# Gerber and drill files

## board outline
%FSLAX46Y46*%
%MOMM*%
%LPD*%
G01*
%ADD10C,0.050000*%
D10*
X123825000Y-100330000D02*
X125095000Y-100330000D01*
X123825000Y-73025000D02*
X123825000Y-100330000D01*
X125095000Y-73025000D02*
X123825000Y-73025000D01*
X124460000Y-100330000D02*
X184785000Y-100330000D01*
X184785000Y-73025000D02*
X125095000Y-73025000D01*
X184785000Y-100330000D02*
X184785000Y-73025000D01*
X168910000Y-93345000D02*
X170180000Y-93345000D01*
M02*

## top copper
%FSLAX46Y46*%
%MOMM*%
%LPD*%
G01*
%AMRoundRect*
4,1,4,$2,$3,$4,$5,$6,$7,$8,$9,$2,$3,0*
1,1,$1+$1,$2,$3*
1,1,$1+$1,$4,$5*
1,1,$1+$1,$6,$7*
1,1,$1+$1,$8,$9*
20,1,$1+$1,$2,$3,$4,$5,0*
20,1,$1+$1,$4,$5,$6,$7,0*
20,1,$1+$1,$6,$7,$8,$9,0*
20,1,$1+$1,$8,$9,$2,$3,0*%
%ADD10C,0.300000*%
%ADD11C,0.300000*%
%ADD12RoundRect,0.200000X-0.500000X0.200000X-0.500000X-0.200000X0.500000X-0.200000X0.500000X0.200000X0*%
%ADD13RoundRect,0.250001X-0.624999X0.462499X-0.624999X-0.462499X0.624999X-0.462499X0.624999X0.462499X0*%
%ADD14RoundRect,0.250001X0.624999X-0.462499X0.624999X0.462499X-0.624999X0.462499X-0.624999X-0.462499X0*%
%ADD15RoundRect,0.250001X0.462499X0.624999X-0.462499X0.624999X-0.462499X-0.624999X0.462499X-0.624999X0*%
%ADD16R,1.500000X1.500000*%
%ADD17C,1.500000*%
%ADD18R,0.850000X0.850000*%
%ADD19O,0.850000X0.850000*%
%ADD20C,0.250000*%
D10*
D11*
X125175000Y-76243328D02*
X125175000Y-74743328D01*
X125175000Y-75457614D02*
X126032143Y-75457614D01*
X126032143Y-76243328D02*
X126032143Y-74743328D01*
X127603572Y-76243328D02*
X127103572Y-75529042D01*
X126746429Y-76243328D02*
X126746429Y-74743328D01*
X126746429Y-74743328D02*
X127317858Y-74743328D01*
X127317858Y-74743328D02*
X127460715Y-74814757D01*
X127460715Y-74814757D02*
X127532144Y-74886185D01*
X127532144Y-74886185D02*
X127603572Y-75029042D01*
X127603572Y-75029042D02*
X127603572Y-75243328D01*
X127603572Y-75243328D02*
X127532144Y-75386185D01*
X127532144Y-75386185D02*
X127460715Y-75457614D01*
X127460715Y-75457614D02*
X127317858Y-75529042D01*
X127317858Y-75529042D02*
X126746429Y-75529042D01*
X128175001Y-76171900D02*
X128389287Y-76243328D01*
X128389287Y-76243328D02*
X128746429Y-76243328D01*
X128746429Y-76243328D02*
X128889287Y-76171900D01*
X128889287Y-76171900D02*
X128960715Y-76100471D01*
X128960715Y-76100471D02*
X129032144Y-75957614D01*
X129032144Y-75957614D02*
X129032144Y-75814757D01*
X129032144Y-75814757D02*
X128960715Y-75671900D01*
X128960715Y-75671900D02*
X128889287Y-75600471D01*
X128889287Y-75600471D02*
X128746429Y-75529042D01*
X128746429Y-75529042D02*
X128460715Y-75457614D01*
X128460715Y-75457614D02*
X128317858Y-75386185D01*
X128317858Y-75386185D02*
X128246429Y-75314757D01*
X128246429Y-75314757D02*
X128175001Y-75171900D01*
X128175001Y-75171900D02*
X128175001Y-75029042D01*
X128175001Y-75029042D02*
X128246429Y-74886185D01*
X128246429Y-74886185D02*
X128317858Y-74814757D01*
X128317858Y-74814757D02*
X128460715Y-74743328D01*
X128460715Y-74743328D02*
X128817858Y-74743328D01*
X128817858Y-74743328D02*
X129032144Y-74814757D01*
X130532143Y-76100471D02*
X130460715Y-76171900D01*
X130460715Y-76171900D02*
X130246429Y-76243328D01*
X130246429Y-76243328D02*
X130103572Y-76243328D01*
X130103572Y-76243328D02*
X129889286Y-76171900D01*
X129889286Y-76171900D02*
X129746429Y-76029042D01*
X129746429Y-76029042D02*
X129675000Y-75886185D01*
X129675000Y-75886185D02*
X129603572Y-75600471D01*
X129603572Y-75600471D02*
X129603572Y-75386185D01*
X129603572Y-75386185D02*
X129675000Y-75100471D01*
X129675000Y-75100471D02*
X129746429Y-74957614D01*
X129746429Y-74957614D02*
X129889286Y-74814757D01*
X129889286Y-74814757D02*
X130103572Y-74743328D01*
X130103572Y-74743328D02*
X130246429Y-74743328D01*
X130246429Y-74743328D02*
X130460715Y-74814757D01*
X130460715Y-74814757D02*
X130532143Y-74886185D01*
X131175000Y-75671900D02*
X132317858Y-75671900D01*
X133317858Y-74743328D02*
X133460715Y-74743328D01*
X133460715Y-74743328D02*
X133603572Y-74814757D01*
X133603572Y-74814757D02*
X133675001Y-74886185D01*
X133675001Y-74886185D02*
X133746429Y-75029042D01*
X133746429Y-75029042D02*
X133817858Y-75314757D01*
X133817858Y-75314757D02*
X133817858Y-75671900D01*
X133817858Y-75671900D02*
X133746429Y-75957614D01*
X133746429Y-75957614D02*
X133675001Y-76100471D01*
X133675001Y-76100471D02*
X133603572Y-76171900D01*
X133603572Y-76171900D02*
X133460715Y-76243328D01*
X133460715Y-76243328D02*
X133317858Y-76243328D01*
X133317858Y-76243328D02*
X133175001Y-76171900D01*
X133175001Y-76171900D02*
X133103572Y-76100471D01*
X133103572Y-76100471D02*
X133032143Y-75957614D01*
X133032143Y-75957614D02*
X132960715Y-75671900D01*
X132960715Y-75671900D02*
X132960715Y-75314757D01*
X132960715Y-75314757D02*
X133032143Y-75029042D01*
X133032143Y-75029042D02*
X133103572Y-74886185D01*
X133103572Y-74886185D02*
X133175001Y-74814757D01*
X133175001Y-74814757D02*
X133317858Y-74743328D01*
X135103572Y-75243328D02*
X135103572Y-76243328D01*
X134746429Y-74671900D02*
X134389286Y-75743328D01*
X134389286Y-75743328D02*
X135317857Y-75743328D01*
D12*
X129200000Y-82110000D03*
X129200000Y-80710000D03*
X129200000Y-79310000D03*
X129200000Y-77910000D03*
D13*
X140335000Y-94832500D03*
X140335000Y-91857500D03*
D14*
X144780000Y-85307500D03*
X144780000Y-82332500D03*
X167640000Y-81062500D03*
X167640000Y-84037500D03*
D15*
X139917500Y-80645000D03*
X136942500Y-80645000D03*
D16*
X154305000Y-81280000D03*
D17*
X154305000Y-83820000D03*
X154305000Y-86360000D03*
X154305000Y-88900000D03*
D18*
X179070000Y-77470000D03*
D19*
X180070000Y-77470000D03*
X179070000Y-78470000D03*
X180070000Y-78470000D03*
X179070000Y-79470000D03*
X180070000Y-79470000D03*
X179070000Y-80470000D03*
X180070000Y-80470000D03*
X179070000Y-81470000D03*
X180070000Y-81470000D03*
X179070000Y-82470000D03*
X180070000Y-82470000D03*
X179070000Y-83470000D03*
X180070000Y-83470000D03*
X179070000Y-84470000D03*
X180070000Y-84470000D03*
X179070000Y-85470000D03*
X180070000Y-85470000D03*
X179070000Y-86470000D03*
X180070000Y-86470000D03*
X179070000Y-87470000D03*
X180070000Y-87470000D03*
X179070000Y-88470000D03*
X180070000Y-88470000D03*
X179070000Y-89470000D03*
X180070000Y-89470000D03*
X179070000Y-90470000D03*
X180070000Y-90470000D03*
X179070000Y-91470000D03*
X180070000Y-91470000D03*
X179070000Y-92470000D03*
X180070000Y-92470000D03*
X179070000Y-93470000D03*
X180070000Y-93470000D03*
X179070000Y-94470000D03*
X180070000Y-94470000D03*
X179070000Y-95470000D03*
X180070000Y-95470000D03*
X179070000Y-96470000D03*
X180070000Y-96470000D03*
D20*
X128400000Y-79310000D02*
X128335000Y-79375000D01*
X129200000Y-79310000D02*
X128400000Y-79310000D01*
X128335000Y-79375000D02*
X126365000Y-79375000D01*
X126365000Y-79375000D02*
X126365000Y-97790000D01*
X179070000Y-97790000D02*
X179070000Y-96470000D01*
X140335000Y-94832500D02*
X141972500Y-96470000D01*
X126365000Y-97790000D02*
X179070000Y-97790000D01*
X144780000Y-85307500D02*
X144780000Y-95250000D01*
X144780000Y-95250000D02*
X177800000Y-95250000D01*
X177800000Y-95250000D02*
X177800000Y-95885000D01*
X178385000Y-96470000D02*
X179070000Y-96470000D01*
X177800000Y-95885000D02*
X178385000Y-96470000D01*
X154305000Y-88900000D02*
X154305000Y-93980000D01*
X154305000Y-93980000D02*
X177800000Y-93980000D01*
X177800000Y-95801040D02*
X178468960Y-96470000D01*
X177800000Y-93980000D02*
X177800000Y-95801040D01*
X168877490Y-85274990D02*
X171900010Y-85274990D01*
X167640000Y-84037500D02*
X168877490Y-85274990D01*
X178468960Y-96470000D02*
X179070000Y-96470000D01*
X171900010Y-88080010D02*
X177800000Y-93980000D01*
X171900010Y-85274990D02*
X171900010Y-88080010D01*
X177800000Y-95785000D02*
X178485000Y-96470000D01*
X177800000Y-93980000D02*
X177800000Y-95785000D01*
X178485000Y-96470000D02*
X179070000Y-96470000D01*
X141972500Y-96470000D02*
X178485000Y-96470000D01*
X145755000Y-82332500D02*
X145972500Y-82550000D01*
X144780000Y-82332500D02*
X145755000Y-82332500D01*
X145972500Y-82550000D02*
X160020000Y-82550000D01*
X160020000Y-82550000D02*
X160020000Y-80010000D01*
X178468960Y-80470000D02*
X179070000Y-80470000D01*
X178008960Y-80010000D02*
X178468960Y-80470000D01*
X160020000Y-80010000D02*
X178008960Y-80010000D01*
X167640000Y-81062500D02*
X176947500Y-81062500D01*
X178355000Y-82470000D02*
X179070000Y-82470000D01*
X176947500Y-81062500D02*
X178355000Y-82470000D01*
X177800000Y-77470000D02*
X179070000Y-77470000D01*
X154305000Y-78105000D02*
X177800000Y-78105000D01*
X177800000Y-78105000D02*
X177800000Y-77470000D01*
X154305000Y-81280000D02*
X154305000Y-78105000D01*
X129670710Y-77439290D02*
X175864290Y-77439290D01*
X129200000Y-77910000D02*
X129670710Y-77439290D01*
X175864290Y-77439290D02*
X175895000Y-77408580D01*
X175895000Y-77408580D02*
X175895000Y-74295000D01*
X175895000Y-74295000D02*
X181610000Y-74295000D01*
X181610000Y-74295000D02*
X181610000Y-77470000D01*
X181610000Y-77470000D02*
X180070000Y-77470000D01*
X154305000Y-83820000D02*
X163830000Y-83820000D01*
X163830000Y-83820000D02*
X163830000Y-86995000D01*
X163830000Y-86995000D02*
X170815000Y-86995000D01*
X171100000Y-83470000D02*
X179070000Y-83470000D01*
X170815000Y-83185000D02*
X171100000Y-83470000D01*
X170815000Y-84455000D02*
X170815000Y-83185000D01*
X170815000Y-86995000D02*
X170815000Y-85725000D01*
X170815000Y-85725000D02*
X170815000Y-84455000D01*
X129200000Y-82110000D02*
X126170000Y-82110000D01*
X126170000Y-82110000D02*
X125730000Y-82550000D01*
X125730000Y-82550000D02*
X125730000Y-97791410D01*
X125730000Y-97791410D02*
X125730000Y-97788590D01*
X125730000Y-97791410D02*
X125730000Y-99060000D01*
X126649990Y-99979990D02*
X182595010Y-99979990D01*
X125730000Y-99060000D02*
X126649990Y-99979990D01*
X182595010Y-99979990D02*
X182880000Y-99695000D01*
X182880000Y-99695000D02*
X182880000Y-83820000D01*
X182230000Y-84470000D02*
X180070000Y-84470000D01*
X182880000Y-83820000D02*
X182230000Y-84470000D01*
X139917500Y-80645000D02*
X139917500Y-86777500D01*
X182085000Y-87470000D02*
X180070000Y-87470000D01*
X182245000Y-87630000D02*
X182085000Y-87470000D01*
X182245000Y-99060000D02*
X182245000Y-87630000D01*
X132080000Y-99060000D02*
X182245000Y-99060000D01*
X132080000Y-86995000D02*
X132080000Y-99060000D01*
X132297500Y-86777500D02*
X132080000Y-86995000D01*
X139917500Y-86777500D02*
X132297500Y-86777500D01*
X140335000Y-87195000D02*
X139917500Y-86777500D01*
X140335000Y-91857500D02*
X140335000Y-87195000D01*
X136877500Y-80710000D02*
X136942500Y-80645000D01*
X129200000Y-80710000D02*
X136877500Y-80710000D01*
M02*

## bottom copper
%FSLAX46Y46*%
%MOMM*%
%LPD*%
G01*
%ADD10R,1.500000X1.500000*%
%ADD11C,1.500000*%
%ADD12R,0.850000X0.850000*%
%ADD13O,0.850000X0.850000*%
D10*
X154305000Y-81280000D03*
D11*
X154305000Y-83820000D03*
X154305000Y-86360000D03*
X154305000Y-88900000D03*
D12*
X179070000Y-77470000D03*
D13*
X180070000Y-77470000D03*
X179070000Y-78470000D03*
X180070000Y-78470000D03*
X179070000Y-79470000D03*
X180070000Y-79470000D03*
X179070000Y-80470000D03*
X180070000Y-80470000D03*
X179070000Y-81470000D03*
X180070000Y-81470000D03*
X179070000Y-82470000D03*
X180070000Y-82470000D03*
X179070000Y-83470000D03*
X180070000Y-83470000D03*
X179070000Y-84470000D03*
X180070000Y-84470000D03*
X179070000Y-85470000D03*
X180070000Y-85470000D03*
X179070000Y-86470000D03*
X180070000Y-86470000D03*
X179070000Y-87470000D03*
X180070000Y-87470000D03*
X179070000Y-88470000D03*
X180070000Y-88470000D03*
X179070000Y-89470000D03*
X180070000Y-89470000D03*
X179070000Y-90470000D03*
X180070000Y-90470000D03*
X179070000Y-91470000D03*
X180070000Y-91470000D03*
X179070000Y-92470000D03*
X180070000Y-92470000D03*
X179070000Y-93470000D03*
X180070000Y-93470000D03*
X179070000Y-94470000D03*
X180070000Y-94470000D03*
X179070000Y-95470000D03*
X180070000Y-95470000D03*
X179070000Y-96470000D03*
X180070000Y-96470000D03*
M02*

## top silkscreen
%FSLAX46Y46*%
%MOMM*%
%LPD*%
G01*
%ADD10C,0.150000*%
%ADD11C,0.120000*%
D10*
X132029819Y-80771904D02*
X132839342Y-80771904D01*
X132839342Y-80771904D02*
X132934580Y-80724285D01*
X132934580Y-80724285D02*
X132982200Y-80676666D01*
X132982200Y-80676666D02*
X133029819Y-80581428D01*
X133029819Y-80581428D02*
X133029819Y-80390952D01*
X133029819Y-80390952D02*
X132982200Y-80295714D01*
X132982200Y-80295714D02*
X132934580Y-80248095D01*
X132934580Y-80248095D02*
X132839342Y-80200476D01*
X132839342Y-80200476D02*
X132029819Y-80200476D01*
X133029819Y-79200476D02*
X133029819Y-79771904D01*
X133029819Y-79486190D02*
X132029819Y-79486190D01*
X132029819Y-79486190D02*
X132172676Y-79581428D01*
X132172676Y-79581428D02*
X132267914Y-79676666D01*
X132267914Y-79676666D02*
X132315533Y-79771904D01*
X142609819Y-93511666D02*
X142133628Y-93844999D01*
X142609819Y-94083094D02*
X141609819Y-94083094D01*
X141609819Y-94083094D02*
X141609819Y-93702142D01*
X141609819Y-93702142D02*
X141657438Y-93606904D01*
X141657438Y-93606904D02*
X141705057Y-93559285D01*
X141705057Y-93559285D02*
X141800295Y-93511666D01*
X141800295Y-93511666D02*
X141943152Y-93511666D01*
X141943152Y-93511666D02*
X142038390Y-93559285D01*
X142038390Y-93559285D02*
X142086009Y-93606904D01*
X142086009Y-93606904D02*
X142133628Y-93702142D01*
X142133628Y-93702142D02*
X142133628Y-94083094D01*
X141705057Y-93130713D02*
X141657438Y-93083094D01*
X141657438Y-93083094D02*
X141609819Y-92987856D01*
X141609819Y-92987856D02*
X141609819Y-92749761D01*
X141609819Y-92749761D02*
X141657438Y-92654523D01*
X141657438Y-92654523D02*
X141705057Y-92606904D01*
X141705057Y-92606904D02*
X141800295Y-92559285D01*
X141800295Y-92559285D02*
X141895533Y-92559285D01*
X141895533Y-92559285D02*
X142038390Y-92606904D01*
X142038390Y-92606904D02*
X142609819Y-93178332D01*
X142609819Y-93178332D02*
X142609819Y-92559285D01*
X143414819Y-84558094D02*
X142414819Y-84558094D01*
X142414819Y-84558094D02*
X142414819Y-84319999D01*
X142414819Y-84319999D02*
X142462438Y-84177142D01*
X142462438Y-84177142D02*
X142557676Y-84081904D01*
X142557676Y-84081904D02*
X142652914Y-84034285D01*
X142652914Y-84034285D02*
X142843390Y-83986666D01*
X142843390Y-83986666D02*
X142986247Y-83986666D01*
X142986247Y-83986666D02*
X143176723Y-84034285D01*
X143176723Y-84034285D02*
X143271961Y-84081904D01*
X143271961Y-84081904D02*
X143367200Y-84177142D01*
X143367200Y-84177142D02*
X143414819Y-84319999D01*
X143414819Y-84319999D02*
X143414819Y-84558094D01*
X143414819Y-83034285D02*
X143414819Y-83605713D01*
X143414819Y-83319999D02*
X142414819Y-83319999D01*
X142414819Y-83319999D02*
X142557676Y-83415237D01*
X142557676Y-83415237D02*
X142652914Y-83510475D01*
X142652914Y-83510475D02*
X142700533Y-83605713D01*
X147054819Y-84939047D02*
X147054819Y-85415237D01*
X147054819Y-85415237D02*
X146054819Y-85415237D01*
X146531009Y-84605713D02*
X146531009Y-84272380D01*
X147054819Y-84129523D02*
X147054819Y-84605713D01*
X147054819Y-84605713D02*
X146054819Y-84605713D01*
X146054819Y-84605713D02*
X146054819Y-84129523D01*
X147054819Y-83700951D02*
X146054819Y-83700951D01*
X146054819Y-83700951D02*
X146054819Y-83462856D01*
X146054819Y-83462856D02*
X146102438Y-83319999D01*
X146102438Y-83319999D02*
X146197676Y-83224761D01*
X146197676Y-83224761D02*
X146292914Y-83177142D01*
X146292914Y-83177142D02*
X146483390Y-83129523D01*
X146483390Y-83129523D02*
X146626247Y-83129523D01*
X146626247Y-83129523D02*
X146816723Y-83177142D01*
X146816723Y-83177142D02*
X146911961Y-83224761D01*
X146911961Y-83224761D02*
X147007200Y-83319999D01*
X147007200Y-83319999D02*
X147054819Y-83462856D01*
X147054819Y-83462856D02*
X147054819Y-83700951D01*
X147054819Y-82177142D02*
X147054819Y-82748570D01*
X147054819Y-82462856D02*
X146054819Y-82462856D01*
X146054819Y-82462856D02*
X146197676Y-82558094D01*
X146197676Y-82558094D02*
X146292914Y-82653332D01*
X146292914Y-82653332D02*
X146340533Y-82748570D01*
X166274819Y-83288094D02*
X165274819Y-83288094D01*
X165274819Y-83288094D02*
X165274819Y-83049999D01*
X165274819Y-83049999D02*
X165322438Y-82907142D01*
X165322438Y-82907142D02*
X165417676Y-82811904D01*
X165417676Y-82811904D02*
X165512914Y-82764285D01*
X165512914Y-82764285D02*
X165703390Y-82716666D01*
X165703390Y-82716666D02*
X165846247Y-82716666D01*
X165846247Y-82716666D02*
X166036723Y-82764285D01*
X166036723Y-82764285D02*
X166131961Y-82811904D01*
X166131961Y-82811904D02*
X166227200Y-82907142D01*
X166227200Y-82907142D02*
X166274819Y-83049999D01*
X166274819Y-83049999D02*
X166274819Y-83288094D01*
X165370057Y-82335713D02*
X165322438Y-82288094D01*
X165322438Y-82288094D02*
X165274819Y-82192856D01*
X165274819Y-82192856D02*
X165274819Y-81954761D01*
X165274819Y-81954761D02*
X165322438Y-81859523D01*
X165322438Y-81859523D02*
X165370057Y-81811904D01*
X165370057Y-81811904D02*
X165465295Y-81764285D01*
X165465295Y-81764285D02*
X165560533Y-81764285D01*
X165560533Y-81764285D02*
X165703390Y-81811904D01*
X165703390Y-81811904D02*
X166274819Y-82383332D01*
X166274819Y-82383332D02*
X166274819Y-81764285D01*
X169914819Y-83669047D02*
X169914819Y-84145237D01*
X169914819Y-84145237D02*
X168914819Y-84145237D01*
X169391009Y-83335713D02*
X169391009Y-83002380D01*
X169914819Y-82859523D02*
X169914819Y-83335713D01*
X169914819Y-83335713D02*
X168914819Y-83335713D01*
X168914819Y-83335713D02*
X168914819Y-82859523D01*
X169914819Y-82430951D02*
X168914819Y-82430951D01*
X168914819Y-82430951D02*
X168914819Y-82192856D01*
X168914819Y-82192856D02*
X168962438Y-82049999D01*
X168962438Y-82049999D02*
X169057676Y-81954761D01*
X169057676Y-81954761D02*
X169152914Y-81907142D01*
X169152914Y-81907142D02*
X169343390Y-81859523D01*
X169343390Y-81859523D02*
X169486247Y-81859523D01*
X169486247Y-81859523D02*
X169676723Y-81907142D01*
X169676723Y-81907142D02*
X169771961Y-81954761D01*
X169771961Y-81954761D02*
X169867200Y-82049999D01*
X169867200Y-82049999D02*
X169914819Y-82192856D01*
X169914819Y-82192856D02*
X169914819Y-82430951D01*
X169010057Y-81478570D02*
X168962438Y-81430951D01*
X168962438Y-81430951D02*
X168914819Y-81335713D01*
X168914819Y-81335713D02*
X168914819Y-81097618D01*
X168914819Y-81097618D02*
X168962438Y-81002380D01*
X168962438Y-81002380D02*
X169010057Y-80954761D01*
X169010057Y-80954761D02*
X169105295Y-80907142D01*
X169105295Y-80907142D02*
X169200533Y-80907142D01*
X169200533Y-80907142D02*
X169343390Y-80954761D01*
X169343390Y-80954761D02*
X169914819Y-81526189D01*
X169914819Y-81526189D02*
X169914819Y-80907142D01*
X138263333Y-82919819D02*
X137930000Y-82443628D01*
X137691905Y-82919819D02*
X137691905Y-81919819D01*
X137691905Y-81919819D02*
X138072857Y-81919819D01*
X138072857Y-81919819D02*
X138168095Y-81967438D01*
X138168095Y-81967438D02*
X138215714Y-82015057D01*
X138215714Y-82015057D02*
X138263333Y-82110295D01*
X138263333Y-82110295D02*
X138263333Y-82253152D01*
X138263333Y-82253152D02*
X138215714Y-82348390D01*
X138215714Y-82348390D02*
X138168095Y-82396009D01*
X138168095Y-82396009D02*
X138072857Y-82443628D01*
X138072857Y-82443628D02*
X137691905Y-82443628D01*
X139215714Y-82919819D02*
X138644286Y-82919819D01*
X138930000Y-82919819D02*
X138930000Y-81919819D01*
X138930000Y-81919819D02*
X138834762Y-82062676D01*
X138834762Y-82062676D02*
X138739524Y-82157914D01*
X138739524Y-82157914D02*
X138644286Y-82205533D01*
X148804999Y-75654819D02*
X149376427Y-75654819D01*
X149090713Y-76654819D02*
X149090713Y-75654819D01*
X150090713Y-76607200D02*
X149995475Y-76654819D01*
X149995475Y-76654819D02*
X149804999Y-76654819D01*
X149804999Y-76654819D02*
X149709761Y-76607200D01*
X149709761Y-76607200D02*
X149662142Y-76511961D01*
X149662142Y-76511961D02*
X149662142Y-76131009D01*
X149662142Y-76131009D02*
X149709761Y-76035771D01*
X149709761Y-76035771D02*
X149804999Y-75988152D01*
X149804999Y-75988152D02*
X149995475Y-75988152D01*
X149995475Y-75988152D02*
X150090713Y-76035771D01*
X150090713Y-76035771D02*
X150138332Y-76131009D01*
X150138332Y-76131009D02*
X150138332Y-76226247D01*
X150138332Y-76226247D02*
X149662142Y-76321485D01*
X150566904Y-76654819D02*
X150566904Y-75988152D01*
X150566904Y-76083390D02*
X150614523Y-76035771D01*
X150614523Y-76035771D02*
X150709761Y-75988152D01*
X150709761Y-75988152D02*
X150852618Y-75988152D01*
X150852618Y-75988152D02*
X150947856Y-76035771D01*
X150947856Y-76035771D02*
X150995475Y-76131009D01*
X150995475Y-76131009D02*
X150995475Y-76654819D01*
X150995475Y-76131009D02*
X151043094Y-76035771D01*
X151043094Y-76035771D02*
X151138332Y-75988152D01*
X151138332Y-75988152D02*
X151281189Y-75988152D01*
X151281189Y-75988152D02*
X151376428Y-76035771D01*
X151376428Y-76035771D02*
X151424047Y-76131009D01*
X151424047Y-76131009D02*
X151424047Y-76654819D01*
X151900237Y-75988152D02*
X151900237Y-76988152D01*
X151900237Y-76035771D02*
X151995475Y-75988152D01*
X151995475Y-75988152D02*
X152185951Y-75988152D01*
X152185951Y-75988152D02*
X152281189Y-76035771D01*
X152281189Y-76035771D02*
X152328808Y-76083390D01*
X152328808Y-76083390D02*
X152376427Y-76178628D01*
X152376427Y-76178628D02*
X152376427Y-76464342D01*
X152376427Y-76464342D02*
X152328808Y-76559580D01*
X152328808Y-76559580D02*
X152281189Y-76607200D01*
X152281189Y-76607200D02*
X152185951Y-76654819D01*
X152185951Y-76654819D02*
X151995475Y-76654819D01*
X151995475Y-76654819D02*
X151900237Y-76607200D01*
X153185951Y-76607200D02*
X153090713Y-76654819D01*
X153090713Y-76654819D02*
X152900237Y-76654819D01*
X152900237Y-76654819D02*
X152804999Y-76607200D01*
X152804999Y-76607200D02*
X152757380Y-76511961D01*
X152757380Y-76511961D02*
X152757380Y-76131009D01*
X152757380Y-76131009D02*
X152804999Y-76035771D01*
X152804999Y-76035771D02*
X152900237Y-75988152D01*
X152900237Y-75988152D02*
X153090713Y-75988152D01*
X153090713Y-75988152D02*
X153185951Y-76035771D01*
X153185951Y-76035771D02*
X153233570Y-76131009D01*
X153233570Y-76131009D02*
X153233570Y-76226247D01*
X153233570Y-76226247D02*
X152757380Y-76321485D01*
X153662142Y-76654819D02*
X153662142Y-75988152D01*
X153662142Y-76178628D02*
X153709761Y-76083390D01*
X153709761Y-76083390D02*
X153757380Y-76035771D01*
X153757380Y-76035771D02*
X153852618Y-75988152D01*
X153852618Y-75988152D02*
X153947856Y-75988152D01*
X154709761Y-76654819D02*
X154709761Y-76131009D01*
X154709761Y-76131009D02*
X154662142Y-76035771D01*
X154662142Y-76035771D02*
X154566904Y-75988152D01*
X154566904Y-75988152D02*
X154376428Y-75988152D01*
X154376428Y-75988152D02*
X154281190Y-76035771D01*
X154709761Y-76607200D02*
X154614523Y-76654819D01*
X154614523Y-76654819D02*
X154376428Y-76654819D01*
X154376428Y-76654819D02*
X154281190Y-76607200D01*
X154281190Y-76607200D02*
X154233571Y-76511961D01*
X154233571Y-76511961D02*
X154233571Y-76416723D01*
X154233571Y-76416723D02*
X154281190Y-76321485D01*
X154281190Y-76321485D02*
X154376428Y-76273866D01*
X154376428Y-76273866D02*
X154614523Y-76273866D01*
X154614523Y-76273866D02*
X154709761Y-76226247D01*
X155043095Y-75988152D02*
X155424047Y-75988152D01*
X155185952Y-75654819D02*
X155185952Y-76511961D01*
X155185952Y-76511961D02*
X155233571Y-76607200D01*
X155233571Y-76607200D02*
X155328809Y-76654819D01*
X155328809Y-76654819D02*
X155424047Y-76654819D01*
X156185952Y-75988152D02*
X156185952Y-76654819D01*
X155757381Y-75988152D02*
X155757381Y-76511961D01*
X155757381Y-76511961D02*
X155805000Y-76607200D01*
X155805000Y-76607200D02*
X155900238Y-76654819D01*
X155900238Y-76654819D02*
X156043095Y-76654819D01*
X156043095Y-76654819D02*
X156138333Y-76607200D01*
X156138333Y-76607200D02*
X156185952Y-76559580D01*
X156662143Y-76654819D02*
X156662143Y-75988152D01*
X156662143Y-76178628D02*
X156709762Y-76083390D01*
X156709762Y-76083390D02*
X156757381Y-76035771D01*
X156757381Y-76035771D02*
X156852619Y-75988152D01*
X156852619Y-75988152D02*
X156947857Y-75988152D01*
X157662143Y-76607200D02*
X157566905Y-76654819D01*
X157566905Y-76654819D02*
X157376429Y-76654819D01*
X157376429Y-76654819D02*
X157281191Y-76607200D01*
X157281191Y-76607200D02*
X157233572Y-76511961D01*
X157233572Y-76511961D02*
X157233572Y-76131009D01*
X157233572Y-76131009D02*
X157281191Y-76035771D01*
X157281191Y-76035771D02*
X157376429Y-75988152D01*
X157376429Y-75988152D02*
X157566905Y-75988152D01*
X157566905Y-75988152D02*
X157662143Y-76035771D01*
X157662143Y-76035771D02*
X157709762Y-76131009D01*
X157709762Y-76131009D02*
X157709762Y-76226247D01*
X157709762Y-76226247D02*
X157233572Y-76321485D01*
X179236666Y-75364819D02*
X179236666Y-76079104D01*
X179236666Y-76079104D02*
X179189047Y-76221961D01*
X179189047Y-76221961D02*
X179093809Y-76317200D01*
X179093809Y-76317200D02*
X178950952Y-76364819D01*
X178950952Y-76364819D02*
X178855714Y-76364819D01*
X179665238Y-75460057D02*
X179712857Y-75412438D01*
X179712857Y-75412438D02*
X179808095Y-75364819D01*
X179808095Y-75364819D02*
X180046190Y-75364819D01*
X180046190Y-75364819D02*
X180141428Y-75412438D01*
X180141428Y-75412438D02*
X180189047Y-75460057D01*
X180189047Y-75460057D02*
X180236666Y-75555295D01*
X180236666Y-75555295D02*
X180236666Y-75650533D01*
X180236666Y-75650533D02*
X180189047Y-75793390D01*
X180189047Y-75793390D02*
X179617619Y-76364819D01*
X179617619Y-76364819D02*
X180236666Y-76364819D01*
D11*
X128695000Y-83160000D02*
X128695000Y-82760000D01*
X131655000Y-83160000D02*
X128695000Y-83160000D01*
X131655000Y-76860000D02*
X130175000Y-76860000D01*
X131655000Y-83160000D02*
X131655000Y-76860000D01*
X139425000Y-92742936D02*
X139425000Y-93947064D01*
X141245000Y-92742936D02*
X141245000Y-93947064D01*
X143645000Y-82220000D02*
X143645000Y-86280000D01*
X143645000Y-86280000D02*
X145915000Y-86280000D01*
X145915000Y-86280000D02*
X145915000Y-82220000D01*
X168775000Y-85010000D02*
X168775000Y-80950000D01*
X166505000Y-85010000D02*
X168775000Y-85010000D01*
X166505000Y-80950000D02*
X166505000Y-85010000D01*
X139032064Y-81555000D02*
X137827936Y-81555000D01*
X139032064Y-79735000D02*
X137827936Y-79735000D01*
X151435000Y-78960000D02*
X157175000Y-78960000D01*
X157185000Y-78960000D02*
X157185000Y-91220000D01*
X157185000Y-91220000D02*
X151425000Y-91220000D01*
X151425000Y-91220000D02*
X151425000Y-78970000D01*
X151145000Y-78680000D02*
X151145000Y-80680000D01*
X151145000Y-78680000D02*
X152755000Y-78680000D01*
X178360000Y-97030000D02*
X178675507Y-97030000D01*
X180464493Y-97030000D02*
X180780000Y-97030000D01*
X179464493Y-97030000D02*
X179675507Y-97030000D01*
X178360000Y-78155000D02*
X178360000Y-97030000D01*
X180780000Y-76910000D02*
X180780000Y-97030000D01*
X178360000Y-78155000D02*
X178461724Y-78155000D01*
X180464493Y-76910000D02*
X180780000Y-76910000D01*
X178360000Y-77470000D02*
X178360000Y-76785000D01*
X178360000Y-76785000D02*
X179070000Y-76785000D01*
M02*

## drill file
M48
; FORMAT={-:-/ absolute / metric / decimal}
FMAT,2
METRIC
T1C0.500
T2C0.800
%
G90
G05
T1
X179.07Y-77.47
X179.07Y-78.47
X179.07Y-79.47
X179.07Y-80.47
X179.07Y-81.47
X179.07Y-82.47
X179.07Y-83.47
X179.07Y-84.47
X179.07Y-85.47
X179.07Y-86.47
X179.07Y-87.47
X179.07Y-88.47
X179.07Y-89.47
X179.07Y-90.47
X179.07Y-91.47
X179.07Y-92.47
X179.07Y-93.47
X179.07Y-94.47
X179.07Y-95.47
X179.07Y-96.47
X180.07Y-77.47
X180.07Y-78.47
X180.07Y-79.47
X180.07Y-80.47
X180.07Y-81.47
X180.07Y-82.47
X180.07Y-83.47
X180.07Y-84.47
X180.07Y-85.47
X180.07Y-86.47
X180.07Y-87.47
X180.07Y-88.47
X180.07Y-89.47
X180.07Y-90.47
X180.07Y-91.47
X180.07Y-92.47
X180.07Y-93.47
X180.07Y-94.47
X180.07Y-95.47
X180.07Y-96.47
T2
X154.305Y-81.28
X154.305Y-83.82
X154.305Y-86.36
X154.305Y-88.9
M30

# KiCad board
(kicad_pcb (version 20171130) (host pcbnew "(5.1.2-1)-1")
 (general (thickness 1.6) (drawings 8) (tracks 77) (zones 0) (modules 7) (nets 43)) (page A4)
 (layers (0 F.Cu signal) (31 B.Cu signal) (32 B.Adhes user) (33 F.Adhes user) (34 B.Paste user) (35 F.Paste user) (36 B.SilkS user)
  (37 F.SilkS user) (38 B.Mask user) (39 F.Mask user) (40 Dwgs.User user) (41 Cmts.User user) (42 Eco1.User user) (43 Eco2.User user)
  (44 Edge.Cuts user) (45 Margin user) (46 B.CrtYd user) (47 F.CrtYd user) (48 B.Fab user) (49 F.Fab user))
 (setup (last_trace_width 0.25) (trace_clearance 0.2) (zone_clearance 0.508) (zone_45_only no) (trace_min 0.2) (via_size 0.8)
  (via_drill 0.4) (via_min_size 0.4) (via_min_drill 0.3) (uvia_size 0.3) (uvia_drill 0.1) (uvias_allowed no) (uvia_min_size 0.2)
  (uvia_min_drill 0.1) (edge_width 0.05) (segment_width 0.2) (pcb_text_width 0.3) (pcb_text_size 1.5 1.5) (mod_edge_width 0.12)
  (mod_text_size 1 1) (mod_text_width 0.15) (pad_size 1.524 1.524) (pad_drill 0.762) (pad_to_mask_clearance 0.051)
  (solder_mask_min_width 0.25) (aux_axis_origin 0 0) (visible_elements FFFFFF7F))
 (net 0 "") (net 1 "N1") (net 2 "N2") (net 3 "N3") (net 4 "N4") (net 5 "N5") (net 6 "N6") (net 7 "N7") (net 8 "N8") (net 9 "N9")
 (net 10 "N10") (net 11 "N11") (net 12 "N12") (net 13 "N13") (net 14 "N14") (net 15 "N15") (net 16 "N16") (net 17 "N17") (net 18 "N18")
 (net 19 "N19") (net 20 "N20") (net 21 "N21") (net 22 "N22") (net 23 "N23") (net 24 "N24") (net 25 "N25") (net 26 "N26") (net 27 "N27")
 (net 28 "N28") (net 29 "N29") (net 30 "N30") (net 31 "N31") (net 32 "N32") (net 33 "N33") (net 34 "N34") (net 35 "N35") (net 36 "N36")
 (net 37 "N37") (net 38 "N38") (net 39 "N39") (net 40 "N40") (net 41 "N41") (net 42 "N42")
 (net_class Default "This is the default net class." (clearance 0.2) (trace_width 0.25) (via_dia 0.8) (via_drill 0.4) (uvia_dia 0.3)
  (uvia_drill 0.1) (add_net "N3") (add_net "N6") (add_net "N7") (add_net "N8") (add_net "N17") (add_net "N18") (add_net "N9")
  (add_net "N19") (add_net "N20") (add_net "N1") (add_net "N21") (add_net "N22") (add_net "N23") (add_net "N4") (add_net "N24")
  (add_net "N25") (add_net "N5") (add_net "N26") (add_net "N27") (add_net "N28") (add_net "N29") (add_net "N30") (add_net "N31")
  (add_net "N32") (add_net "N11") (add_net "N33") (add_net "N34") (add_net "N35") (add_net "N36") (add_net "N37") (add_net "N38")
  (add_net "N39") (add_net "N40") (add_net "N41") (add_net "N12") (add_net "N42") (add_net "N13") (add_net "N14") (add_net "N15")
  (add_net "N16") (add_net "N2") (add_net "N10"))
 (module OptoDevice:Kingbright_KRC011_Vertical (layer F.Cu) (at 130.175 80.01 270)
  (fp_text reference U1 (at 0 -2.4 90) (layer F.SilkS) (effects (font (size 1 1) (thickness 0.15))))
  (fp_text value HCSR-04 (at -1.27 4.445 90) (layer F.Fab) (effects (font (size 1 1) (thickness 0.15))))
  (fp_line (start 3.15 1.48) (end 2.75 1.48) (layer F.SilkS) (width 0.12))
  (fp_line (start 3.15 -1.48) (end 3.15 1.48) (layer F.SilkS) (width 0.12))
  (fp_line (start -3.15 -1.48) (end -3.15 0) (layer F.SilkS) (width 0.12))
  (fp_line (start 3.15 -1.48) (end -3.15 -1.48) (layer F.SilkS) (width 0.12))
  (pad 4 smd roundrect (at 2.1 0.975 270) (size 0.8 1.4) (layers F.Cu F.Paste F.Mask) (roundrect_rratio 0.25) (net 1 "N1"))
  (pad 3 smd roundrect (at 0.7 0.975 270) (size 0.8 1.4) (layers F.Cu F.Paste F.Mask) (roundrect_rratio 0.25) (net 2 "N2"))
  (pad 2 smd roundrect (at -0.7 0.975 270) (size 0.8 1.4) (layers F.Cu F.Paste F.Mask) (roundrect_rratio 0.25) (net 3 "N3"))
  (pad 1 smd roundrect (at -2.1 0.975 270) (size 0.8 1.4) (layers F.Cu F.Paste F.Mask) (roundrect_rratio 0.25) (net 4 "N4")))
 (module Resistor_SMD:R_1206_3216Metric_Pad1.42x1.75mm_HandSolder (layer F.Cu) (at 140.335 93.345 270)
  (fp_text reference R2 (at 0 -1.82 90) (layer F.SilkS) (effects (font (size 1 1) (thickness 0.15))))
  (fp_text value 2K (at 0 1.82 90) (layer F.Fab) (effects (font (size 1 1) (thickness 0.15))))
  (fp_line (start -0.602064 0.91) (end 0.602064 0.91) (layer F.SilkS) (width 0.12))
  (fp_line (start -0.602064 -0.91) (end 0.602064 -0.91) (layer F.SilkS) (width 0.12))
  (pad 2 smd roundrect (at 1.4875 0 270) (size 1.425 1.75) (layers F.Cu F.Paste F.Mask) (roundrect_rratio 0.175439) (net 3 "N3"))
  (pad 1 smd roundrect (at -1.4875 0 270) (size 1.425 1.75) (layers F.Cu F.Paste F.Mask) (roundrect_rratio 0.175439) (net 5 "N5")))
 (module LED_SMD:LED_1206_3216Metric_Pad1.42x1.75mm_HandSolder (layer F.Cu) (at 144.78 83.82 90)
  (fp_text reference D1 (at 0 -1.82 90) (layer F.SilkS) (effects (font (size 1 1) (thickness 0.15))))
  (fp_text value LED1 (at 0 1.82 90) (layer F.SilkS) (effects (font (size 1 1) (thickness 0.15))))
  (fp_line (start 1.6 -1.135) (end -2.46 -1.135) (layer F.SilkS) (width 0.12))
  (fp_line (start -2.46 -1.135) (end -2.46 1.135) (layer F.SilkS) (width 0.12))
  (fp_line (start -2.46 1.135) (end 1.6 1.135) (layer F.SilkS) (width 0.12))
  (pad 1 smd roundrect (at -1.4875 0 90) (size 1.425 1.75) (layers F.Cu F.Paste F.Mask) (roundrect_rratio 0.175439) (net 3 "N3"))
  (pad 2 smd roundrect (at 1.4875 0 90) (size 1.425 1.75) (layers F.Cu F.Paste F.Mask) (roundrect_rratio 0.175439) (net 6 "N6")))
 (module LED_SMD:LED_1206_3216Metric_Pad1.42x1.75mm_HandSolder (layer F.Cu) (at 167.64 82.55 90)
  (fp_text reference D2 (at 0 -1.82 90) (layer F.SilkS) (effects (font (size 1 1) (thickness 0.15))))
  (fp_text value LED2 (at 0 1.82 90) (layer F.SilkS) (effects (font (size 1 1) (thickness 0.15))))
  (fp_line (start -2.46 1.135) (end 1.6 1.135) (layer F.SilkS) (width 0.12))
  (fp_line (start -2.46 -1.135) (end -2.46 1.135) (layer F.SilkS) (width 0.12))
  (fp_line (start 1.6 -1.135) (end -2.46 -1.135) (layer F.SilkS) (width 0.12))
  (pad 2 smd roundrect (at 1.4875 0 90) (size 1.425 1.75) (layers F.Cu F.Paste F.Mask) (roundrect_rratio 0.175439) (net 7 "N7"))
  (pad 1 smd roundrect (at -1.4875 0 90) (size 1.425 1.75) (layers F.Cu F.Paste F.Mask) (roundrect_rratio 0.175439) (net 3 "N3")))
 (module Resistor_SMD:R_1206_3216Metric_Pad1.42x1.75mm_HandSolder (layer F.Cu) (at 138.43 80.645 180)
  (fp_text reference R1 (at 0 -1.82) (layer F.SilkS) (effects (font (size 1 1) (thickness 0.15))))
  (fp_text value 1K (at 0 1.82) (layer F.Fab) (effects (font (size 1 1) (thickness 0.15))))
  (fp_line (start -0.602064 -0.91) (end 0.602064 -0.91) (layer F.SilkS) (width 0.12))
  (fp_line (start -0.602064 0.91) (end 0.602064 0.91) (layer F.SilkS) (width 0.12))
  (pad 1 smd roundrect (at -1.4875 0 180) (size 1.425 1.75) (layers F.Cu F.Paste F.Mask) (roundrect_rratio 0.175439) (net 5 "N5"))
  (pad 2 smd roundrect (at 1.4875 0 180) (size 1.425 1.75) (layers F.Cu F.Paste F.Mask) (roundrect_rratio 0.175439) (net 2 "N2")))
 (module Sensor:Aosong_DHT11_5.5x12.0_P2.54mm (layer F.Cu) (at 154.305 81.28)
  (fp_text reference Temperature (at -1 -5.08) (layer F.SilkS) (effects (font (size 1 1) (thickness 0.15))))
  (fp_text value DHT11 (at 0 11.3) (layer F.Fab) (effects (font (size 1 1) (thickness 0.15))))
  (fp_line (start -2.87 -2.32) (end 2.87 -2.32) (layer F.SilkS) (width 0.12))
  (fp_line (start 2.88 -2.32) (end 2.88 9.94) (layer F.SilkS) (width 0.12))
  (fp_line (start 2.88 9.94) (end -2.88 9.94) (layer F.SilkS) (width 0.12))
  (fp_line (start -2.88 9.94) (end -2.88 -2.31) (layer F.SilkS) (width 0.12))
  (fp_line (start -3.16 -2.6) (end -3.16 -0.6) (layer F.SilkS) (width 0.12))
  (fp_line (start -3.16 -2.6) (end -1.55 -2.6) (layer F.SilkS) (width 0.12))
  (pad 1 thru_hole rect (at 0 0) (size 1.5 1.5) (drill 0.8) (layers *.Cu *.Mask) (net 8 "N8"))
  (pad 2 thru_hole circle (at 0 2.54) (size 1.5 1.5) (drill 0.8) (layers *.Cu *.Mask) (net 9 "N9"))
  (pad 3 thru_hole circle (at 0 5.08) (size 1.5 1.5) (drill 0.8) (layers *.Cu *.Mask) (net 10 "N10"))
  (pad 4 thru_hole circle (at 0 7.62) (size 1.5 1.5) (drill 0.8) (layers *.Cu *.Mask) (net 3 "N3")))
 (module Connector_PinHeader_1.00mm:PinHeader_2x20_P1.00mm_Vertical (layer F.Cu) (at 179.07 77.47)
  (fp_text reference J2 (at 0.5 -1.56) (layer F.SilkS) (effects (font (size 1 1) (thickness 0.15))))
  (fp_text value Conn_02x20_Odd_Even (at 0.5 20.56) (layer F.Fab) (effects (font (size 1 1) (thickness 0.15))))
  (fp_line (start -0.71 19.56) (end -0.394493 19.56) (layer F.SilkS) (width 0.12))
  (fp_line (start 1.394493 19.56) (end 1.71 19.56) (layer F.SilkS) (width 0.12))
  (fp_line (start 0.394493 19.56) (end 0.605507 19.56) (layer F.SilkS) (width 0.12))
  (fp_line (start -0.71 0.685) (end -0.71 19.56) (layer F.SilkS) (width 0.12))
  (fp_line (start 1.71 -0.56) (end 1.71 19.56) (layer F.SilkS) (width 0.12))
  (fp_line (start -0.71 0.685) (end -0.608276 0.685) (layer F.SilkS) (width 0.12))
  (fp_line (start 1.394493 -0.56) (end 1.71 -0.56) (layer F.SilkS) (width 0.12))
  (fp_line (start -0.71 0) (end -0.71 -0.685) (layer F.SilkS) (width 0.12))
  (fp_line (start -0.71 -0.685) (end 0 -0.685) (layer F.SilkS) (width 0.12))
  (pad 1 thru_hole rect (at 0 0) (size 0.85 0.85) (drill 0.5) (layers *.Cu *.Mask) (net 8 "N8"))
  (pad 2 thru_hole oval (at 1 0) (size 0.85 0.85) (drill 0.5) (layers *.Cu *.Mask) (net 4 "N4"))
  (pad 3 thru_hole oval (at 0 1) (size 0.85 0.85) (drill 0.5) (layers *.Cu *.Mask) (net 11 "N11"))
  (pad 4 thru_hole oval (at 1 1) (size 0.85 0.85) (drill 0.5) (layers *.Cu *.Mask) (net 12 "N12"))
  (pad 5 thru_hole oval (at 0 2) (size 0.85 0.85) (drill 0.5) (layers *.Cu *.Mask) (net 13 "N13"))
  (pad 6 thru_hole oval (at 1 2) (size 0.85 0.85) (drill 0.5) (layers *.Cu *.Mask) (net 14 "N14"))
  (pad 7 thru_hole oval (at 0 3) (size 0.85 0.85) (drill 0.5) (layers *.Cu *.Mask) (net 6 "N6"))
  (pad 8 thru_hole oval (at 1 3) (size 0.85 0.85) (drill 0.5) (layers *.Cu *.Mask) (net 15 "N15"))
  (pad 9 thru_hole oval (at 0 4) (size 0.85 0.85) (drill 0.5) (layers *.Cu *.Mask) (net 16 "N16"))
  (pad 10 thru_hole oval (at 1 4) (size 0.85 0.85) (drill 0.5) (layers *.Cu *.Mask) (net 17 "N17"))
  (pad 11 thru_hole oval (at 0 5) (size 0.85 0.85) (drill 0.5) (layers *.Cu *.Mask) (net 7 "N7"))
  (pad 12 thru_hole oval (at 1 5) (size 0.85 0.85) (drill 0.5) (layers *.Cu *.Mask) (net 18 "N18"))
  (pad 13 thru_hole oval (at 0 6) (size 0.85 0.85) (drill 0.5) (layers *.Cu *.Mask) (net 9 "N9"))
  (pad 14 thru_hole oval (at 1 6) (size 0.85 0.85) (drill 0.5) (layers *.Cu *.Mask) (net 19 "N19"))
  (pad 15 thru_hole oval (at 0 7) (size 0.85 0.85) (drill 0.5) (layers *.Cu *.Mask) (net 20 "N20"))
  (pad 16 thru_hole oval (at 1 7) (size 0.85 0.85) (drill 0.5) (layers *.Cu *.Mask) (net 1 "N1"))
  (pad 17 thru_hole oval (at 0 8) (size 0.85 0.85) (drill 0.5) (layers *.Cu *.Mask) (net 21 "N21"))
  (pad 18 thru_hole oval (at 1 8) (size 0.85 0.85) (drill 0.5) (layers *.Cu *.Mask) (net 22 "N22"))
  (pad 19 thru_hole oval (at 0 9) (size 0.85 0.85) (drill 0.5) (layers *.Cu *.Mask) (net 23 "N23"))
  (pad 20 thru_hole oval (at 1 9) (size 0.85 0.85) (drill 0.5) (layers *.Cu *.Mask) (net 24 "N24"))
  (pad 21 thru_hole oval (at 0 10) (size 0.85 0.85) (drill 0.5) (layers *.Cu *.Mask) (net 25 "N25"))
  (pad 22 thru_hole oval (at 1 10) (size 0.85 0.85) (drill 0.5) (layers *.Cu *.Mask) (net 5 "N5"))
  (pad 23 thru_hole oval (at 0 11) (size 0.85 0.85) (drill 0.5) (layers *.Cu *.Mask) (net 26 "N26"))
  (pad 24 thru_hole oval (at 1 11) (size 0.85 0.85) (drill 0.5) (layers *.Cu *.Mask) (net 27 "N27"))
  (pad 25 thru_hole oval (at 0 12) (size 0.85 0.85) (drill 0.5) (layers *.Cu *.Mask) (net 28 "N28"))
  (pad 26 thru_hole oval (at 1 12) (size 0.85 0.85) (drill 0.5) (layers *.Cu *.Mask) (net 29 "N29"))
  (pad 27 thru_hole oval (at 0 13) (size 0.85 0.85) (drill 0.5) (layers *.Cu *.Mask) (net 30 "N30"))
  (pad 28 thru_hole oval (at 1 13) (size 0.85 0.85) (drill 0.5) (layers *.Cu *.Mask) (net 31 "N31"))
  (pad 29 thru_hole oval (at 0 14) (size 0.85 0.85) (drill 0.5) (layers *.Cu *.Mask) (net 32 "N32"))
  (pad 30 thru_hole oval (at 1 14) (size 0.85 0.85) (drill 0.5) (layers *.Cu *.Mask) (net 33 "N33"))
  (pad 31 thru_hole oval (at 0 15) (size 0.85 0.85) (drill 0.5) (layers *.Cu *.Mask) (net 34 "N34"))
  (pad 32 thru_hole oval (at 1 15) (size 0.85 0.85) (drill 0.5) (layers *.Cu *.Mask) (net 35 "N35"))
  (pad 33 thru_hole oval (at 0 16) (size 0.85 0.85) (drill 0.5) (layers *.Cu *.Mask) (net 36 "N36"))
  (pad 34 thru_hole oval (at 1 16) (size 0.85 0.85) (drill 0.5) (layers *.Cu *.Mask) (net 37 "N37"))
  (pad 35 thru_hole oval (at 0 17) (size 0.85 0.85) (drill 0.5) (layers *.Cu *.Mask) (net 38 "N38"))
  (pad 36 thru_hole oval (at 1 17) (size 0.85 0.85) (drill 0.5) (layers *.Cu *.Mask) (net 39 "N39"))
  (pad 37 thru_hole oval (at 0 18) (size 0.85 0.85) (drill 0.5) (layers *.Cu *.Mask) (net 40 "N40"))
  (pad 38 thru_hole oval (at 1 18) (size 0.85 0.85) (drill 0.5) (layers *.Cu *.Mask) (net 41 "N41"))
  (pad 39 thru_hole oval (at 0 19) (size 0.85 0.85) (drill 0.5) (layers *.Cu *.Mask) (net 3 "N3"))
  (pad 40 thru_hole oval (at 1 19) (size 0.85 0.85) (drill 0.5) (layers *.Cu *.Mask) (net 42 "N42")))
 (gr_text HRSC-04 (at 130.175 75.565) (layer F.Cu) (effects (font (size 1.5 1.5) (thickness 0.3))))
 (gr_line (start 123.825 100.33) (end 125.095 100.33) (layer Edge.Cuts) (width 0.05))
 (gr_line (start 123.825 73.025) (end 123.825 100.33) (layer Edge.Cuts) (width 0.05))
 (gr_line (start 125.095 73.025) (end 123.825 73.025) (layer Edge.Cuts) (width 0.05))
 (gr_line (start 124.46 100.33) (end 184.785 100.33) (layer Edge.Cuts) (width 0.05))
 (gr_line (start 184.785 73.025) (end 125.095 73.025) (layer Edge.Cuts) (width 0.05))
 (gr_line (start 184.785 100.33) (end 184.785 73.025) (layer Edge.Cuts) (width 0.05))
 (gr_line (start 168.91 93.345) (end 170.18 93.345) (layer Edge.Cuts) (width 0.05))
 (segment (start 128.4 79.31) (end 128.335 79.375) (width 0.25) (layer F.Cu) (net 3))
 (segment (start 129.2 79.31) (end 128.4 79.31) (width 0.25) (layer F.Cu) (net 3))
 (segment (start 128.335 79.375) (end 126.365 79.375) (width 0.25) (layer F.Cu) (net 3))
 (segment (start 126.365 79.375) (end 126.365 97.79) (width 0.25) (layer F.Cu) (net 3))
 (segment (start 179.07 97.79) (end 179.07 96.47) (width 0.25) (layer F.Cu) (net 3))
 (segment (start 140.335 94.8325) (end 141.9725 96.47) (width 0.25) (layer F.Cu) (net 3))
 (segment (start 126.365 97.79) (end 179.07 97.79) (width 0.25) (layer F.Cu) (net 3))
 (segment (start 144.78 85.3075) (end 144.78 95.25) (width 0.25) (layer F.Cu) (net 3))
 (segment (start 144.78 95.25) (end 177.8 95.25) (width 0.25) (layer F.Cu) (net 3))
 (segment (start 177.8 95.25) (end 177.8 95.885) (width 0.25) (layer F.Cu) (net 3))
 (segment (start 178.385 96.47) (end 179.07 96.47) (width 0.25) (layer F.Cu) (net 3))
 (segment (start 177.8 95.885) (end 178.385 96.47) (width 0.25) (layer F.Cu) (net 3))
 (segment (start 154.305 88.9) (end 154.305 93.98) (width 0.25) (layer F.Cu) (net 3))
 (segment (start 154.305 93.98) (end 177.8 93.98) (width 0.25) (layer F.Cu) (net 3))
 (segment (start 177.8 95.80104) (end 178.46896 96.47) (width 0.25) (layer F.Cu) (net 3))
 (segment (start 177.8 93.98) (end 177.8 95.80104) (width 0.25) (layer F.Cu) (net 3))
 (segment (start 168.87749 85.27499) (end 171.90001 85.27499) (width 0.25) (layer F.Cu) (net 3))
 (segment (start 167.64 84.0375) (end 168.87749 85.27499) (width 0.25) (layer F.Cu) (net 3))
 (segment (start 178.46896 96.47) (end 179.07 96.47) (width 0.25) (layer F.Cu) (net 3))
 (segment (start 171.90001 88.08001) (end 177.8 93.98) (width 0.25) (layer F.Cu) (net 3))
 (segment (start 171.90001 85.27499) (end 171.90001 88.08001) (width 0.25) (layer F.Cu) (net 3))
 (segment (start 177.8 95.785) (end 178.485 96.47) (width 0.25) (layer F.Cu) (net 3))
 (segment (start 177.8 93.98) (end 177.8 95.785) (width 0.25) (layer F.Cu) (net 3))
 (segment (start 178.485 96.47) (end 179.07 96.47) (width 0.25) (layer F.Cu) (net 3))
 (segment (start 141.9725 96.47) (end 178.485 96.47) (width 0.25) (layer F.Cu) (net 3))
 (segment (start 145.755 82.3325) (end 145.9725 82.55) (width 0.25) (layer F.Cu) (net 6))
 (segment (start 144.78 82.3325) (end 145.755 82.3325) (width 0.25) (layer F.Cu) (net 6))
 (segment (start 145.9725 82.55) (end 160.02 82.55) (width 0.25) (layer F.Cu) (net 6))
 (segment (start 160.02 82.55) (end 160.02 80.01) (width 0.25) (layer F.Cu) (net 6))
 (segment (start 178.46896 80.47) (end 179.07 80.47) (width 0.25) (layer F.Cu) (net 6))
 (segment (start 178.00896 80.01) (end 178.46896 80.47) (width 0.25) (layer F.Cu) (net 6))
 (segment (start 160.02 80.01) (end 178.00896 80.01) (width 0.25) (layer F.Cu) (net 6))
 (segment (start 167.64 81.0625) (end 176.9475 81.0625) (width 0.25) (layer F.Cu) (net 7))
 (segment (start 178.355 82.47) (end 179.07 82.47) (width 0.25) (layer F.Cu) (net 7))
 (segment (start 176.9475 81.0625) (end 178.355 82.47) (width 0.25) (layer F.Cu) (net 7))
 (segment (start 177.8 77.47) (end 179.07 77.47) (width 0.25) (layer F.Cu) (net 8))
 (segment (start 154.305 78.105) (end 177.8 78.105) (width 0.25) (layer F.Cu) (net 8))
 (segment (start 177.8 78.105) (end 177.8 77.47) (width 0.25) (layer F.Cu) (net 8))
 (segment (start 154.305 81.28) (end 154.305 78.105) (width 0.25) (layer F.Cu) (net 8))
 (segment (start 129.67071 77.43929) (end 175.86429 77.43929) (width 0.25) (layer F.Cu) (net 4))
 (segment (start 129.2 77.91) (end 129.67071 77.43929) (width 0.25) (layer F.Cu) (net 4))
 (segment (start 175.86429 77.43929) (end 175.895 77.40858) (width 0.25) (layer F.Cu) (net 4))
 (segment (start 175.895 77.40858) (end 175.895 74.295) (width 0.25) (layer F.Cu) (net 4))
 (segment (start 175.895 74.295) (end 181.61 74.295) (width 0.25) (layer F.Cu) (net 4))
 (segment (start 181.61 74.295) (end 181.61 77.47) (width 0.25) (layer F.Cu) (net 4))
 (segment (start 181.61 77.47) (end 180.07 77.47) (width 0.25) (layer F.Cu) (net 4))
 (segment (start 154.305 83.82) (end 163.83 83.82) (width 0.25) (layer F.Cu) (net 9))
 (segment (start 163.83 83.82) (end 163.83 86.995) (width 0.25) (layer F.Cu) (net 9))
 (segment (start 163.83 86.995) (end 170.815 86.995) (width 0.25) (layer F.Cu) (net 9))
 (segment (start 171.1 83.47) (end 179.07 83.47) (width 0.25) (layer F.Cu) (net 9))
 (segment (start 170.815 83.185) (end 171.1 83.47) (width 0.25) (layer F.Cu) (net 9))
 (segment (start 170.815 84.455) (end 170.815 83.185) (width 0.25) (layer F.Cu) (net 9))
 (segment (start 170.815 86.995) (end 170.815 85.725) (width 0.25) (layer F.Cu) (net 9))
 (segment (start 170.815 85.725) (end 170.815 84.455) (width 0.25) (layer F.Cu) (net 9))
 (segment (start 129.2 82.11) (end 126.17 82.11) (width 0.25) (layer F.Cu) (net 1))
 (segment (start 126.17 82.11) (end 125.73 82.55) (width 0.25) (layer F.Cu) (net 1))
 (segment (start 125.73 82.55) (end 125.73 97.79141) (width 0.25) (layer F.Cu) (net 1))
 (segment (start 125.73 97.79141) (end 125.73 97.78859) (width 0.25) (layer F.Cu) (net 1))
 (segment (start 125.73 97.79141) (end 125.73 99.06) (width 0.25) (layer F.Cu) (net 1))
 (segment (start 126.64999 99.97999) (end 182.59501 99.97999) (width 0.25) (layer F.Cu) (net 1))
 (segment (start 125.73 99.06) (end 126.64999 99.97999) (width 0.25) (layer F.Cu) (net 1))
 (segment (start 182.59501 99.97999) (end 182.88 99.695) (width 0.25) (layer F.Cu) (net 1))
 (segment (start 182.88 99.695) (end 182.88 83.82) (width 0.25) (layer F.Cu) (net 1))
 (segment (start 182.23 84.47) (end 180.07 84.47) (width 0.25) (layer F.Cu) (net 1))
 (segment (start 182.88 83.82) (end 182.23 84.47) (width 0.25) (layer F.Cu) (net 1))
 (segment (start 139.9175 80.645) (end 139.9175 86.7775) (width 0.25) (layer F.Cu) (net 5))
 (segment (start 182.085 87.47) (end 180.07 87.47) (width 0.25) (layer F.Cu) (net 5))
 (segment (start 182.245 87.63) (end 182.085 87.47) (width 0.25) (layer F.Cu) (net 5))
 (segment (start 182.245 99.06) (end 182.245 87.63) (width 0.25) (layer F.Cu) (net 5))
 (segment (start 132.08 99.06) (end 182.245 99.06) (width 0.25) (layer F.Cu) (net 5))
 (segment (start 132.08 86.995) (end 132.08 99.06) (width 0.25) (layer F.Cu) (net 5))
 (segment (start 132.2975 86.7775) (end 132.08 86.995) (width 0.25) (layer F.Cu) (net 5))
 (segment (start 139.9175 86.7775) (end 132.2975 86.7775) (width 0.25) (layer F.Cu) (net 5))
 (segment (start 140.335 87.195) (end 139.9175 86.7775) (width 0.25) (layer F.Cu) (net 5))
 (segment (start 140.335 91.8575) (end 140.335 87.195) (width 0.25) (layer F.Cu) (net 5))
 (segment (start 136.8775 80.71) (end 136.9425 80.645) (width 0.25) (layer F.Cu) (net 2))
 (segment (start 129.2 80.71) (end 136.8775 80.71) (width 0.25) (layer F.Cu) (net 2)))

